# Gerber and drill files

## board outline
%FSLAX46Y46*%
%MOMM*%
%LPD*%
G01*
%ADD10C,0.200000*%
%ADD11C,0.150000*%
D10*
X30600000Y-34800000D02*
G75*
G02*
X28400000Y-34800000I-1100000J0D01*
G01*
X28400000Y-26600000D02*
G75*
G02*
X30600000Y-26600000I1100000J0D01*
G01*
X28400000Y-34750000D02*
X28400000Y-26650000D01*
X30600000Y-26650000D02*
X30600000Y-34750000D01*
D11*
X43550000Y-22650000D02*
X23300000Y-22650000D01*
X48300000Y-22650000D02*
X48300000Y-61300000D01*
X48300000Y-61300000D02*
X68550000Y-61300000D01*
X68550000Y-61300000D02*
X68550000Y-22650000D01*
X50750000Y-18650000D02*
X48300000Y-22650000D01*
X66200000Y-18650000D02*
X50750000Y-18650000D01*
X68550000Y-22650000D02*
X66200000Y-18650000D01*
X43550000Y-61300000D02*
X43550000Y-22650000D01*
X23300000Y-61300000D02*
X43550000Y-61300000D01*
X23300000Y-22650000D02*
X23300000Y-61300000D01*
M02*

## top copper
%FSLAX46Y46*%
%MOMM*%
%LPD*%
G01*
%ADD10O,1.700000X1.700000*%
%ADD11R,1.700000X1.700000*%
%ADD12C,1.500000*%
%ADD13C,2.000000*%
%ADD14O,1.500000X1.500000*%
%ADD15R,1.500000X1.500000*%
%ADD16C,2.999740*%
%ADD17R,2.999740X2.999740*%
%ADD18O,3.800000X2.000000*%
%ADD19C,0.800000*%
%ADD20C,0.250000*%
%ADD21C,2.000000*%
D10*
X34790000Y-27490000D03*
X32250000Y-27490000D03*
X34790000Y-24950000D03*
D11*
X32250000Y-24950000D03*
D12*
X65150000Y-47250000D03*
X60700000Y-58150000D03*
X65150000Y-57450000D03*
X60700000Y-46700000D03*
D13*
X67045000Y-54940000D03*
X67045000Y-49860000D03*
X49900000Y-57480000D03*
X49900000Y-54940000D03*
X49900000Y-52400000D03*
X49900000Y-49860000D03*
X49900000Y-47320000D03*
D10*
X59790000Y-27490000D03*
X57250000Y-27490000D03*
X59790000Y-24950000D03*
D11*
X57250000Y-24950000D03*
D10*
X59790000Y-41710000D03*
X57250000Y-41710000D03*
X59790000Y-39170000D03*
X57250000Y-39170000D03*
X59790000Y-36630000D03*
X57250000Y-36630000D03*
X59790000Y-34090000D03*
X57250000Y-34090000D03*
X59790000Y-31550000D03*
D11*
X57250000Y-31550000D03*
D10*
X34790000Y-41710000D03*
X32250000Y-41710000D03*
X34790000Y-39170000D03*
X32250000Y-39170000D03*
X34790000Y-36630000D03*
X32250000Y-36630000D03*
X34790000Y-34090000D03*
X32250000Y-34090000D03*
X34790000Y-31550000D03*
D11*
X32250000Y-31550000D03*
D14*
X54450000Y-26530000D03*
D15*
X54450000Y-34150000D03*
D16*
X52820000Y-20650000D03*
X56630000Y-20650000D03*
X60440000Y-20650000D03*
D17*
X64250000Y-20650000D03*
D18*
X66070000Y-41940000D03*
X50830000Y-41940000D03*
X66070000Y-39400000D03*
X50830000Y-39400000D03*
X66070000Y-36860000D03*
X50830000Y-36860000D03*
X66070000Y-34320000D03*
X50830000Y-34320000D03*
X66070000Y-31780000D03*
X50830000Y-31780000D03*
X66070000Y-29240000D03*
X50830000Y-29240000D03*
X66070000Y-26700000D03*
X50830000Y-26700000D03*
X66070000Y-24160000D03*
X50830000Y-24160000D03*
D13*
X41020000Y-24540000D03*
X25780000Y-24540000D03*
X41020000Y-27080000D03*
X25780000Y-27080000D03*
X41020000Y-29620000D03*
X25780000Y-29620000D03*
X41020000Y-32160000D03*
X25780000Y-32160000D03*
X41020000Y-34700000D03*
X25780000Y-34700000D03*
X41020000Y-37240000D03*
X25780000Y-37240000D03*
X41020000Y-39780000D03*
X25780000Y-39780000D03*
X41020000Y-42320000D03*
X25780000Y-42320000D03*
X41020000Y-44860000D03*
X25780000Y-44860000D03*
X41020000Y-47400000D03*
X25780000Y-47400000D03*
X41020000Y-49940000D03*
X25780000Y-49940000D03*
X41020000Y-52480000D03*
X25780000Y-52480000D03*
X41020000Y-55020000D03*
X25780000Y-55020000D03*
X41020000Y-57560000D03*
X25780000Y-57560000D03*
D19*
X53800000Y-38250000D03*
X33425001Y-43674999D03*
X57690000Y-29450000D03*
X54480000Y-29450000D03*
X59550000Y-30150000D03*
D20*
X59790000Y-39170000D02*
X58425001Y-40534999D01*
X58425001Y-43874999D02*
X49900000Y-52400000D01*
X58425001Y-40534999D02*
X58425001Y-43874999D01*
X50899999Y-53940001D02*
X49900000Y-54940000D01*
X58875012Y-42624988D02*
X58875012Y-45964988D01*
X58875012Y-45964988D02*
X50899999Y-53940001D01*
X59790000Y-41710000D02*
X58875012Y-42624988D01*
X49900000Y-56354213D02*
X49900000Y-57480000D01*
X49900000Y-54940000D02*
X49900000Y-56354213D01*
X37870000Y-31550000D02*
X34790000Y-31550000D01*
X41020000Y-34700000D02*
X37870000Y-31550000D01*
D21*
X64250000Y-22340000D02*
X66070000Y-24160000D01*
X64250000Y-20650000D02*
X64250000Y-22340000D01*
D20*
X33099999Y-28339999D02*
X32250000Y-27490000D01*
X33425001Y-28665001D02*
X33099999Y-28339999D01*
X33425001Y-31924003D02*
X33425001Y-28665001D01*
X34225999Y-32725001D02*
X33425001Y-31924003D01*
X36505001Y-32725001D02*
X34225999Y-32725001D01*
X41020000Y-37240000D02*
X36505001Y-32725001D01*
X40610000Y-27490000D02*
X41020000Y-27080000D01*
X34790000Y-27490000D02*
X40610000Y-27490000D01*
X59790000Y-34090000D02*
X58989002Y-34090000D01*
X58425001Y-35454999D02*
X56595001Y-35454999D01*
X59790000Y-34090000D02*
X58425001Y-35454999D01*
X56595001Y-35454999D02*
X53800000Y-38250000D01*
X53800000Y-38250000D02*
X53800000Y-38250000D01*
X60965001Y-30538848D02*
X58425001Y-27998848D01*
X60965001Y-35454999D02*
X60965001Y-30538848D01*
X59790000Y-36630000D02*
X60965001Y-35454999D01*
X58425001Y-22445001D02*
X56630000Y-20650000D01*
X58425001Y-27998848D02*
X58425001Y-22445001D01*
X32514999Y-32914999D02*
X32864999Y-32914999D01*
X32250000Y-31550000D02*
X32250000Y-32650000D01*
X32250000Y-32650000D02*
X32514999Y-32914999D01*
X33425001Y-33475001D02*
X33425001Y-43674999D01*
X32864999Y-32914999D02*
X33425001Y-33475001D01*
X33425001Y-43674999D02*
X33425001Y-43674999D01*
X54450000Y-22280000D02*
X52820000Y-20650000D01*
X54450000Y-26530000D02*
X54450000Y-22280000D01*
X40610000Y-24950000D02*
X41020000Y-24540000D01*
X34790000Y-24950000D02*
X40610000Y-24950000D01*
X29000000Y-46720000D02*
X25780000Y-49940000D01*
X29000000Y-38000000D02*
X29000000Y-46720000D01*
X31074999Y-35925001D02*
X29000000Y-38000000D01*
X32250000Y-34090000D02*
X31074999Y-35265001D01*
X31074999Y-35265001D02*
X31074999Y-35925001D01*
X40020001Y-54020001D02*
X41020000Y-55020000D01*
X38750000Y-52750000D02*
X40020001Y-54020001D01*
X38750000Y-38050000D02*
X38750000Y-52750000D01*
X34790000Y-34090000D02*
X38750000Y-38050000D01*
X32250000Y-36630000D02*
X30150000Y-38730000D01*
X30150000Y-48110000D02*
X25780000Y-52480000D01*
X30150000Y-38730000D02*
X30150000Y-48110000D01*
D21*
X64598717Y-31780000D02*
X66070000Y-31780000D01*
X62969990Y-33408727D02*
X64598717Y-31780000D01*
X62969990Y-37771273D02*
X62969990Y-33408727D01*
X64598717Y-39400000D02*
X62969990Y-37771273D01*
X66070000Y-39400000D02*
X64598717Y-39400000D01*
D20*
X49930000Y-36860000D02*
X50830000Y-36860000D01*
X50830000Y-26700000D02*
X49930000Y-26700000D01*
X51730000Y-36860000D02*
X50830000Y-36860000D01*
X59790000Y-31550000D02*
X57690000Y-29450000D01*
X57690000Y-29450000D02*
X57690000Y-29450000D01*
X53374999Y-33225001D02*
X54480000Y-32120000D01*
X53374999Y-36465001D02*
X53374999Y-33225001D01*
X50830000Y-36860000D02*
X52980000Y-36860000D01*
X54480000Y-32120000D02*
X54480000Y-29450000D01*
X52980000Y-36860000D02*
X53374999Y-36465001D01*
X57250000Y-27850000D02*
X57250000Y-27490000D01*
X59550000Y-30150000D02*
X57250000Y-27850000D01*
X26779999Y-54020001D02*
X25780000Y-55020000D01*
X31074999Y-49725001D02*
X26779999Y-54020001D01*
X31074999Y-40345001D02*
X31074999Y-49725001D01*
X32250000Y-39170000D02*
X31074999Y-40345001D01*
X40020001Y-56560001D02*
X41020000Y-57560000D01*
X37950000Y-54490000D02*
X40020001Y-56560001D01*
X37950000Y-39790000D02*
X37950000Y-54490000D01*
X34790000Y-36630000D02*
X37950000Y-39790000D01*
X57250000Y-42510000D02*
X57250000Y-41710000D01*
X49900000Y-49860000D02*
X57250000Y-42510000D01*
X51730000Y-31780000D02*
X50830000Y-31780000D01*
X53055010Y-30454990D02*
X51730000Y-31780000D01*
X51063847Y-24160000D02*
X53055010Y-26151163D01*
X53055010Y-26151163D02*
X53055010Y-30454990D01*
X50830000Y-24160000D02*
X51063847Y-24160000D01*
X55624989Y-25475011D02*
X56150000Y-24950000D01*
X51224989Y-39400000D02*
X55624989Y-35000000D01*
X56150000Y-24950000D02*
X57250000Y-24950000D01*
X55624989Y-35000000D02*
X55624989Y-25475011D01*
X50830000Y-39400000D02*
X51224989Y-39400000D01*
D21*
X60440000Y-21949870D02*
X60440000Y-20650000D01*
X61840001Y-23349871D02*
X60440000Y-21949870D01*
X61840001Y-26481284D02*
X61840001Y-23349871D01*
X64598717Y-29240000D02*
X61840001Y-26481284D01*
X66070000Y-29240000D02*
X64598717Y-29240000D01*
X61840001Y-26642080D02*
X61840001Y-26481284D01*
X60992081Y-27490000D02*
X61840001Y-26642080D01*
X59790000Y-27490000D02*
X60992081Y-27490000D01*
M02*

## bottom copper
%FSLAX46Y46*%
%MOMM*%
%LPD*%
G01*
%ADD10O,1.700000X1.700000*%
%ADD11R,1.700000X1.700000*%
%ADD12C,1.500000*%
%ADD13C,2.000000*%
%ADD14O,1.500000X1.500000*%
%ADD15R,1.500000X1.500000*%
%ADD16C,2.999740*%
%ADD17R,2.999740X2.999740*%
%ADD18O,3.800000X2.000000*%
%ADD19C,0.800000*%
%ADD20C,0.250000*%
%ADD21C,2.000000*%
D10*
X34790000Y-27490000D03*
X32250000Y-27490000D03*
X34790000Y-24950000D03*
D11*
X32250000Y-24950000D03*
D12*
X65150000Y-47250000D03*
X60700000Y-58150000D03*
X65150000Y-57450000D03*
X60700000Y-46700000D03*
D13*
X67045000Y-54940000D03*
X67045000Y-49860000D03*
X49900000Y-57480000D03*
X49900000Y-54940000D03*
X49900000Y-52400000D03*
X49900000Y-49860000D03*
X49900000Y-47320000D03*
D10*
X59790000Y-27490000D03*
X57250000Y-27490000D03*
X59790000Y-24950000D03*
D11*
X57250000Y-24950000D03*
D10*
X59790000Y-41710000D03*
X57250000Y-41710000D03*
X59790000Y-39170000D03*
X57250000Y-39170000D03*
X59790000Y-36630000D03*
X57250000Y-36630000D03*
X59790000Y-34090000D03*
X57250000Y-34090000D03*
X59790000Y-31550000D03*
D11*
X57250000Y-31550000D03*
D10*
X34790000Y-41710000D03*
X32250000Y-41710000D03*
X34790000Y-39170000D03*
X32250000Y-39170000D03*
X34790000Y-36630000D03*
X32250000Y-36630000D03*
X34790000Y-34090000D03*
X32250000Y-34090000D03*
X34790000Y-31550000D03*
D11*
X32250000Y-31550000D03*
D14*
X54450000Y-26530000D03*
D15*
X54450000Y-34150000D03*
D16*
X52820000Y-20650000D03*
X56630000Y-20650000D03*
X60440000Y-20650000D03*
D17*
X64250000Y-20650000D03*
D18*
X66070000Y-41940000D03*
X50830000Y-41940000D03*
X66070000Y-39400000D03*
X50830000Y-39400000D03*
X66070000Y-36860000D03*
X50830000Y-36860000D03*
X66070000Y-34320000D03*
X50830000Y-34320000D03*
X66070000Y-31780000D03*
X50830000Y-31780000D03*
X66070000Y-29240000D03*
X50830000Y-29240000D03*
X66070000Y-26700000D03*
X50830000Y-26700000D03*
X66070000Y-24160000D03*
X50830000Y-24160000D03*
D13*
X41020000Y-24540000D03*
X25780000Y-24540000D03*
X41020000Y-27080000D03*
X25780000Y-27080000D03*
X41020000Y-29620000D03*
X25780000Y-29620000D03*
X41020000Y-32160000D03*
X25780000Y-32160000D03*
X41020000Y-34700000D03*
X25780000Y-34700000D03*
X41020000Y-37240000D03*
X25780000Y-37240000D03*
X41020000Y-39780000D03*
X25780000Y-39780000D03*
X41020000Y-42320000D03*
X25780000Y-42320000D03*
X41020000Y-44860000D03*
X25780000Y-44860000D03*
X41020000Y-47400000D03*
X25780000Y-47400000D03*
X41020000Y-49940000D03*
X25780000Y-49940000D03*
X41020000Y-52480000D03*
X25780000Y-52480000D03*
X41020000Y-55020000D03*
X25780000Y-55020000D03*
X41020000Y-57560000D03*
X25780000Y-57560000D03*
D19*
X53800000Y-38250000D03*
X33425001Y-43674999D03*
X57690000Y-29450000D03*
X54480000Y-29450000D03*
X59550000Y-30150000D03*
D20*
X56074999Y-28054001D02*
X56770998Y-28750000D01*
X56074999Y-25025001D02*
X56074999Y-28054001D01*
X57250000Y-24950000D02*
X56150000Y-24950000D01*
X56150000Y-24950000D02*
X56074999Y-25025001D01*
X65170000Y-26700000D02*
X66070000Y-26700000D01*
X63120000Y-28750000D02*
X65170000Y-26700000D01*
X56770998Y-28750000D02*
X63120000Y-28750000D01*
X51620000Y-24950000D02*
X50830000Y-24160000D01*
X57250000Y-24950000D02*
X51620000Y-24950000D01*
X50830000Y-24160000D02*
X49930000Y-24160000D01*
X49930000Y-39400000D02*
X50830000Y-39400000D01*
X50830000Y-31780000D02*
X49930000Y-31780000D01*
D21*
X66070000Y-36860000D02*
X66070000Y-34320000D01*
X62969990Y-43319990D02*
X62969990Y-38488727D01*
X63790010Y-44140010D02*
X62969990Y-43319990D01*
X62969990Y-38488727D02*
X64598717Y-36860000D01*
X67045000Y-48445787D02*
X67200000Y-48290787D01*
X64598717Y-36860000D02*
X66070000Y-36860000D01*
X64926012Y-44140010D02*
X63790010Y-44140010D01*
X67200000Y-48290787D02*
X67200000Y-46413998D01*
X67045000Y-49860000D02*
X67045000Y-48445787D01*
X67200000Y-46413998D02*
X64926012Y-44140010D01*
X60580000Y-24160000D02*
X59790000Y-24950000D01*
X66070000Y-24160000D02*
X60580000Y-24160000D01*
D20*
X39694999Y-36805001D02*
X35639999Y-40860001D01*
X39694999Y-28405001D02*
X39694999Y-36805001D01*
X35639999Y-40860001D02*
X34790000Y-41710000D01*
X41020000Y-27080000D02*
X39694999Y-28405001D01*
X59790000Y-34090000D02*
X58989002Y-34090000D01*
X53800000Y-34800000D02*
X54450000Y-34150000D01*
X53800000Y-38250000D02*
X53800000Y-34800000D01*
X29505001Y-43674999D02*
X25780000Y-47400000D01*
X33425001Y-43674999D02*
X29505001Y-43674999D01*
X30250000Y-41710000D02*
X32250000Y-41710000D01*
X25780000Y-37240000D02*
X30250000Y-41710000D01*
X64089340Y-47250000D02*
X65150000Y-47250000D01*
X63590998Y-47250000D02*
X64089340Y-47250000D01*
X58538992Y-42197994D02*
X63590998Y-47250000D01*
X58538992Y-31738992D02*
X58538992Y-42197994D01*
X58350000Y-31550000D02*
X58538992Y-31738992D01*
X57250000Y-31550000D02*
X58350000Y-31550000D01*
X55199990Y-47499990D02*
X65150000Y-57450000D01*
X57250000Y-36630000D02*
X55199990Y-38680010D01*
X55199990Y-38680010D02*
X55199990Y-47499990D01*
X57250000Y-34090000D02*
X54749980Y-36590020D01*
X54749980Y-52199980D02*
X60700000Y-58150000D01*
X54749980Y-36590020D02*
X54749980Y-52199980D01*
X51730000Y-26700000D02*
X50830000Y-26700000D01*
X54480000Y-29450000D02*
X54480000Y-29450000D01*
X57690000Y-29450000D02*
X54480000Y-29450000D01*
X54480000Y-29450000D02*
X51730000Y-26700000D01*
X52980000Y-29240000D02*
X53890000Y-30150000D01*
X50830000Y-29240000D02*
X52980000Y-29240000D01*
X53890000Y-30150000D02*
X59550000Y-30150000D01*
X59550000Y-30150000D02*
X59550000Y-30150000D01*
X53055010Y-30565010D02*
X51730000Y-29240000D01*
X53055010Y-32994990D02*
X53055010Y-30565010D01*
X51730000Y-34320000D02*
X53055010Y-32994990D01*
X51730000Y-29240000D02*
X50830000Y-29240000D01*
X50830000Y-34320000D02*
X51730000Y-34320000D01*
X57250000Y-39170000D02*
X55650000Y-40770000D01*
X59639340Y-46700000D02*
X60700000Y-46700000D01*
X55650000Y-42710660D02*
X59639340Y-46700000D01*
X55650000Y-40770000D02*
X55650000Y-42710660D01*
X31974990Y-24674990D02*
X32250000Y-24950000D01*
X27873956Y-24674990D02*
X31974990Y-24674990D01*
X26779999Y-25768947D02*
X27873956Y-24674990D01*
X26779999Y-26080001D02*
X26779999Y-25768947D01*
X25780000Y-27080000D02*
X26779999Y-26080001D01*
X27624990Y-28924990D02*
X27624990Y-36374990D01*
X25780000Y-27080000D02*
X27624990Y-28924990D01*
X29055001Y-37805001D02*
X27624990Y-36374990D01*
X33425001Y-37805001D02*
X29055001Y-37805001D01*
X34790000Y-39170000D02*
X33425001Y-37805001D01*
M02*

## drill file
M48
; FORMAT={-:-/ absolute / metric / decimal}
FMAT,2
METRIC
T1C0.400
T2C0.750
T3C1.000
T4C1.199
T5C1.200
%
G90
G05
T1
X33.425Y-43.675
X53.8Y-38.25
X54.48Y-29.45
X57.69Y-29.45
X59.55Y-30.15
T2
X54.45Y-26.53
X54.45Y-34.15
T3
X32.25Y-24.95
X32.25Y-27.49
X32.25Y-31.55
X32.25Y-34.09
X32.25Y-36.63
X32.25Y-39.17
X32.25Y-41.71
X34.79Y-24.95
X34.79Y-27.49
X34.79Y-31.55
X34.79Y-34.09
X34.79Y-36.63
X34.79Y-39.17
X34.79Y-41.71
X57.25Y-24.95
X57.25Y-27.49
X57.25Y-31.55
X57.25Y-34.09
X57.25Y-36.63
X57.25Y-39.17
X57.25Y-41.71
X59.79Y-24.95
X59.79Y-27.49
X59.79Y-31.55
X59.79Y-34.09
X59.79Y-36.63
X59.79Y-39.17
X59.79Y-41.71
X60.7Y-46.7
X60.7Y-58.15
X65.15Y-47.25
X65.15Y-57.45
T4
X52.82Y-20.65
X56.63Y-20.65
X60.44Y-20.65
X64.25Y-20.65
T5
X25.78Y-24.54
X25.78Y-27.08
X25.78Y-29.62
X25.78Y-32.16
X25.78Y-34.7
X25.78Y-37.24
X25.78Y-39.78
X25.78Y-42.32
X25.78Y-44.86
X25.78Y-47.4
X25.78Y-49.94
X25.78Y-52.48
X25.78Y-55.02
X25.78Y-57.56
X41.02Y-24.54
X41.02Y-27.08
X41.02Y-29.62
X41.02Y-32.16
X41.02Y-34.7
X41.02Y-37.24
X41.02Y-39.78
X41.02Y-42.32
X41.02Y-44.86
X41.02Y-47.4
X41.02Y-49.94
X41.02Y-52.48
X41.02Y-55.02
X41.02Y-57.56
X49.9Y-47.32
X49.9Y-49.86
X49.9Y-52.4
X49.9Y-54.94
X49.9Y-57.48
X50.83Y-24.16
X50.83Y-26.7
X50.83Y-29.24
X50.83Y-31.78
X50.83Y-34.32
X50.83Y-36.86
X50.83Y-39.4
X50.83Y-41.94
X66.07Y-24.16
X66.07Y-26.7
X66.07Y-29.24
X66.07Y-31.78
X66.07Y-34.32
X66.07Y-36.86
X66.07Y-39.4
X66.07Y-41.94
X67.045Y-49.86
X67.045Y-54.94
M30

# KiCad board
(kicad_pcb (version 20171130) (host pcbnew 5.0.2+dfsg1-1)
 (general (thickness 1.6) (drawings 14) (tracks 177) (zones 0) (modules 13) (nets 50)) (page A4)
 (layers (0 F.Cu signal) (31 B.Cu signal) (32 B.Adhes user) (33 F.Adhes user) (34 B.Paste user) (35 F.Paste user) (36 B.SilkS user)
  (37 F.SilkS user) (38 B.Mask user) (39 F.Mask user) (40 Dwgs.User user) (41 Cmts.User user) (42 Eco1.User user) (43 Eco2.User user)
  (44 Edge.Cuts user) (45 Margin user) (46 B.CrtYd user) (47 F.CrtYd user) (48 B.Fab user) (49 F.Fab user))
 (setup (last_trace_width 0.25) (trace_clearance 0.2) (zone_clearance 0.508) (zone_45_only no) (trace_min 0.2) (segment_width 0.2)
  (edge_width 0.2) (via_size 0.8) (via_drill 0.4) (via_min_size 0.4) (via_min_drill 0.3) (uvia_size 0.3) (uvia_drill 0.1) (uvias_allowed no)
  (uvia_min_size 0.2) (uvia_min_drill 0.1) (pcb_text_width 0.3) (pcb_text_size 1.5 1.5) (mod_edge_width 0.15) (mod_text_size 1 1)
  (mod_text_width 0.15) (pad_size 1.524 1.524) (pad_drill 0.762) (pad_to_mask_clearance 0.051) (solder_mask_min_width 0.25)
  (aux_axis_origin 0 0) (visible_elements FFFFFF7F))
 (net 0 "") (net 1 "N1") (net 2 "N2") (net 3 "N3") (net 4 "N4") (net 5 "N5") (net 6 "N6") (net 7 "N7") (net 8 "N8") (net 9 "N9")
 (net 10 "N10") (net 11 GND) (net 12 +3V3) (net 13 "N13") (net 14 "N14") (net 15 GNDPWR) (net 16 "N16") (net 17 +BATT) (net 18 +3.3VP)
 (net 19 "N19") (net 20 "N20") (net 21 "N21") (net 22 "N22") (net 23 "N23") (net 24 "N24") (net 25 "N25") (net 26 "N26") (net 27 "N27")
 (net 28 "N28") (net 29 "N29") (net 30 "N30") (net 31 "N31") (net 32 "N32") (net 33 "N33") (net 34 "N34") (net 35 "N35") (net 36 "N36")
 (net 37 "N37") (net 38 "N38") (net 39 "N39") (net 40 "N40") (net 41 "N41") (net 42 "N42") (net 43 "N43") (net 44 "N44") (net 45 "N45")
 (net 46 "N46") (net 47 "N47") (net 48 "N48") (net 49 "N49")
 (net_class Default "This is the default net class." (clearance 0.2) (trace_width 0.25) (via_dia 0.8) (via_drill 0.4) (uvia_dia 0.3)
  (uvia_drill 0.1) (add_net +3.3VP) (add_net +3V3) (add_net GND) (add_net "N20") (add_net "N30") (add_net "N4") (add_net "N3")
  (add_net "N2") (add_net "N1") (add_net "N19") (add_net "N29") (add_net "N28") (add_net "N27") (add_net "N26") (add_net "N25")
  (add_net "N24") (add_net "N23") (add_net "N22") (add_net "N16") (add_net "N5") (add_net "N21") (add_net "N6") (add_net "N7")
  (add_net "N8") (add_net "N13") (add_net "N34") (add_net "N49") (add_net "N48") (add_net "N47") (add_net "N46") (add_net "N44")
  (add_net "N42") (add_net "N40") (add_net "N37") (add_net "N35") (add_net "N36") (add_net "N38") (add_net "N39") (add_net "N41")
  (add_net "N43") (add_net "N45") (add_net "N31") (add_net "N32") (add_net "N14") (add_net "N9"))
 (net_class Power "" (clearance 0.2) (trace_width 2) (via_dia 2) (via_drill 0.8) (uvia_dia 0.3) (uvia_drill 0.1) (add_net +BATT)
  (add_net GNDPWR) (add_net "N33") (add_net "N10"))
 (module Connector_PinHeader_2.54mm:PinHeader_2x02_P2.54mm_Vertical (layer F.Cu) (at 32.25 24.95)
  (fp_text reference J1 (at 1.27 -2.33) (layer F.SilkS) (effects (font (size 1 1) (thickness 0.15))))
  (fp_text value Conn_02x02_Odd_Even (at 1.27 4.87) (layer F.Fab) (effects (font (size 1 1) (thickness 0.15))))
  (pad 4 thru_hole oval (at 2.54 2.54) (size 1.7 1.7) (drill 1) (layers *.Cu *.Mask) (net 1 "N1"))
  (pad 3 thru_hole oval (at 0 2.54) (size 1.7 1.7) (drill 1) (layers *.Cu *.Mask) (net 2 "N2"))
  (pad 2 thru_hole oval (at 2.54 0) (size 1.7 1.7) (drill 1) (layers *.Cu *.Mask) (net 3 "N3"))
  (pad 1 thru_hole rect (at 0 0) (size 1.7 1.7) (drill 1) (layers *.Cu *.Mask) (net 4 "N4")))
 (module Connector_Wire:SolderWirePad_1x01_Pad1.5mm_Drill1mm (layer B.Cu) (at 65.15 47.25)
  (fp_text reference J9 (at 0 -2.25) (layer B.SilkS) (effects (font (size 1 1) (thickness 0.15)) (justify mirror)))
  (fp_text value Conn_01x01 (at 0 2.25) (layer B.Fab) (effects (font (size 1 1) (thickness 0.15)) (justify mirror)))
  (pad 1 thru_hole circle (at 0 0) (size 1.5 1.5) (drill 1) (layers *.Cu *.Mask) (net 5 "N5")))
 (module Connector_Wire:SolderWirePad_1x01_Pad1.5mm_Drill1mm (layer B.Cu) (at 60.7 58.15)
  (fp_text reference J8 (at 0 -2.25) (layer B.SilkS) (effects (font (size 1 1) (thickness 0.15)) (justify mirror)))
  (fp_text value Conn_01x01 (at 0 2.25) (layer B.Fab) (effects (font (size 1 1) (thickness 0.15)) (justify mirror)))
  (pad 1 thru_hole circle (at 0 0) (size 1.5 1.5) (drill 1) (layers *.Cu *.Mask) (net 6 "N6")))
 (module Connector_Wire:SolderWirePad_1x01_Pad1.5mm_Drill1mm (layer B.Cu) (at 65.15 57.45)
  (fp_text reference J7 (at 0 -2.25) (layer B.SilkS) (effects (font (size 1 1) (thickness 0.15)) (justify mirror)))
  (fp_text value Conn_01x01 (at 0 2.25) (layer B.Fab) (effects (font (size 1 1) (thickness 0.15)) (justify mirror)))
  (pad 1 thru_hole circle (at 0 0) (size 1.5 1.5) (drill 1) (layers *.Cu *.Mask) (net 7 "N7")))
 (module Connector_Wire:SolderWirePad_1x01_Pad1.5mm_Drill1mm (layer B.Cu) (at 60.7 46.7)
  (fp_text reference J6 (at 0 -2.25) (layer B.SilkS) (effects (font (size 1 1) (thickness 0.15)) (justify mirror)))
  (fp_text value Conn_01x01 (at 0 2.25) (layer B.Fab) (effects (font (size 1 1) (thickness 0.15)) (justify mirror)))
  (pad 1 thru_hole circle (at 0 0) (size 1.5 1.5) (drill 1) (layers *.Cu *.Mask) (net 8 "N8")))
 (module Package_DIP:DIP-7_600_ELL (layer B.Cu) (at 49.9 52.4 270)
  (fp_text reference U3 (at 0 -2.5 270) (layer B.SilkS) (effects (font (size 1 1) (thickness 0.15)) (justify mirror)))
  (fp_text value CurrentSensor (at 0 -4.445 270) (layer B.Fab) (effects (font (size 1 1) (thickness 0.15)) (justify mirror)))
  (pad 7 thru_hole circle (at 2.54 -17.145 270) (size 2 2) (drill 1.2) (layers *.Cu *.Mask) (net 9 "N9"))
  (pad 6 thru_hole circle (at -2.54 -17.145 270) (size 2 2) (drill 1.2) (layers *.Cu *.Mask) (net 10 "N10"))
  (pad 5 thru_hole circle (at 5.08 0 270) (size 2 2) (drill 1.2) (layers *.Cu *.Mask) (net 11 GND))
  (pad 4 thru_hole circle (at 2.54 0 270) (size 2 2) (drill 1.2) (layers *.Cu *.Mask) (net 11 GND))
  (pad 3 thru_hole circle (at 0 0 270) (size 2 2) (drill 1.2) (layers *.Cu *.Mask) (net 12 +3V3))
  (pad 2 thru_hole circle (at -2.54 0 270) (size 2 2) (drill 1.2) (layers *.Cu *.Mask) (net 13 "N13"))
  (pad 1 thru_hole circle (at -5.08 0 270) (size 2 2) (drill 1.2) (layers *.Cu *.Mask) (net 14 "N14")))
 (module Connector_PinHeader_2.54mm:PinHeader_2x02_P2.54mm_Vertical (layer F.Cu) (at 57.25 24.95)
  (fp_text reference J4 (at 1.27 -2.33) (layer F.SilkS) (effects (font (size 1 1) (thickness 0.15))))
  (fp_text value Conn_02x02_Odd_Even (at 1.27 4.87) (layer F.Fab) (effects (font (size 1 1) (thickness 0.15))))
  (pad 4 thru_hole oval (at 2.54 2.54) (size 1.7 1.7) (drill 1) (layers *.Cu *.Mask) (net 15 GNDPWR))
  (pad 3 thru_hole oval (at 0 2.54) (size 1.7 1.7) (drill 1) (layers *.Cu *.Mask) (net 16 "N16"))
  (pad 2 thru_hole oval (at 2.54 0) (size 1.7 1.7) (drill 1) (layers *.Cu *.Mask) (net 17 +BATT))
  (pad 1 thru_hole rect (at 0 0) (size 1.7 1.7) (drill 1) (layers *.Cu *.Mask) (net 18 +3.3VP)))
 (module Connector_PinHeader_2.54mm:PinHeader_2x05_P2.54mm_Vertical (layer F.Cu) (at 57.25 31.55)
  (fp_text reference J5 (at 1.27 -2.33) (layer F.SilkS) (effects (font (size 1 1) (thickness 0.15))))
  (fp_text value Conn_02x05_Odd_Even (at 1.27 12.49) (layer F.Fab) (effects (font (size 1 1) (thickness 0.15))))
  (pad 10 thru_hole oval (at 2.54 10.16) (size 1.7 1.7) (drill 1) (layers *.Cu *.Mask) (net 11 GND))
  (pad 9 thru_hole oval (at 0 10.16) (size 1.7 1.7) (drill 1) (layers *.Cu *.Mask) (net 13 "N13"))
  (pad 8 thru_hole oval (at 2.54 7.62) (size 1.7 1.7) (drill 1) (layers *.Cu *.Mask) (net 12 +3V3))
  (pad 7 thru_hole oval (at 0 7.62) (size 1.7 1.7) (drill 1) (layers *.Cu *.Mask) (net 8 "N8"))
  (pad 6 thru_hole oval (at 2.54 5.08) (size 1.7 1.7) (drill 1) (layers *.Cu *.Mask) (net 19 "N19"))
  (pad 5 thru_hole oval (at 0 5.08) (size 1.7 1.7) (drill 1) (layers *.Cu *.Mask) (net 7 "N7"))
  (pad 4 thru_hole oval (at 2.54 2.54) (size 1.7 1.7) (drill 1) (layers *.Cu *.Mask) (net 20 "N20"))
  (pad 3 thru_hole oval (at 0 2.54) (size 1.7 1.7) (drill 1) (layers *.Cu *.Mask) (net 6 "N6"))
  (pad 2 thru_hole oval (at 2.54 0) (size 1.7 1.7) (drill 1) (layers *.Cu *.Mask) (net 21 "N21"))
  (pad 1 thru_hole rect (at 0 0) (size 1.7 1.7) (drill 1) (layers *.Cu *.Mask) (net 5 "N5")))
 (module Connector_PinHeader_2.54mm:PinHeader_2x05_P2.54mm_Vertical (layer F.Cu) (at 32.25 31.55)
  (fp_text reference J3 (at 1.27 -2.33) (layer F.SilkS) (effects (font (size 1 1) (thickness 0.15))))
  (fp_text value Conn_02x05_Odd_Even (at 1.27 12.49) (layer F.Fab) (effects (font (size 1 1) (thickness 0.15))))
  (pad 10 thru_hole oval (at 2.54 10.16) (size 1.7 1.7) (drill 1) (layers *.Cu *.Mask) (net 1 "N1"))
  (pad 9 thru_hole oval (at 0 10.16) (size 1.7 1.7) (drill 1) (layers *.Cu *.Mask) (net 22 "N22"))
  (pad 8 thru_hole oval (at 2.54 7.62) (size 1.7 1.7) (drill 1) (layers *.Cu *.Mask) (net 4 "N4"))
  (pad 7 thru_hole oval (at 0 7.62) (size 1.7 1.7) (drill 1) (layers *.Cu *.Mask) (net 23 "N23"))
  (pad 6 thru_hole oval (at 2.54 5.08) (size 1.7 1.7) (drill 1) (layers *.Cu *.Mask) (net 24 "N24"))
  (pad 5 thru_hole oval (at 0 5.08) (size 1.7 1.7) (drill 1) (layers *.Cu *.Mask) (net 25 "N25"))
  (pad 4 thru_hole oval (at 2.54 2.54) (size 1.7 1.7) (drill 1) (layers *.Cu *.Mask) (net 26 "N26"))
  (pad 3 thru_hole oval (at 0 2.54) (size 1.7 1.7) (drill 1) (layers *.Cu *.Mask) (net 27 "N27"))
  (pad 2 thru_hole oval (at 2.54 0) (size 1.7 1.7) (drill 1) (layers *.Cu *.Mask) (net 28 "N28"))
  (pad 1 thru_hole rect (at 0 0) (size 1.7 1.7) (drill 1) (layers *.Cu *.Mask) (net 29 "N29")))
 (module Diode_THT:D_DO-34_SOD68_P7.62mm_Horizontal (layer F.Cu) (at 54.45 34.15 90)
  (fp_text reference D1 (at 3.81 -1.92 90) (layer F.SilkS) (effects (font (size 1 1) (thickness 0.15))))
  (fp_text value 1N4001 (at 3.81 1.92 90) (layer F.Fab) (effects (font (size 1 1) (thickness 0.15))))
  (pad 2 thru_hole oval (at 7.62 0 90) (size 1.5 1.5) (drill 0.75) (layers *.Cu *.Mask) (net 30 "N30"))
  (pad 1 thru_hole rect (at 0 0 90) (size 1.5 1.5) (drill 0.75) (layers *.Cu *.Mask) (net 20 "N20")))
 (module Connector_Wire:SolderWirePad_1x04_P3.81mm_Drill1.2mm (layer F.Cu) (at 64.25 20.65 180)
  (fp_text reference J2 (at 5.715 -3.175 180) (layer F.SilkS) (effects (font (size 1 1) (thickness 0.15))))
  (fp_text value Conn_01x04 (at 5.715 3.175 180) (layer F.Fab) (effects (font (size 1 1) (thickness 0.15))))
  (pad 4 thru_hole circle (at 11.43 0 180) (size 2.99974 2.99974) (drill 1.19888) (layers *.Cu *.Mask) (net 30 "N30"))
  (pad 3 thru_hole circle (at 7.62 0 180) (size 2.99974 2.99974) (drill 1.19888) (layers *.Cu *.Mask) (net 19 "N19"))
  (pad 2 thru_hole circle (at 3.81 0 180) (size 2.99974 2.99974) (drill 1.19888) (layers *.Cu *.Mask) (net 15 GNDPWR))
  (pad 1 thru_hole rect (at 0 0 180) (size 2.99974 2.99974) (drill 1.19888) (layers *.Cu *.Mask) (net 17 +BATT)))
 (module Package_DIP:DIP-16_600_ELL (layer B.Cu) (at 58.45 33.05 270)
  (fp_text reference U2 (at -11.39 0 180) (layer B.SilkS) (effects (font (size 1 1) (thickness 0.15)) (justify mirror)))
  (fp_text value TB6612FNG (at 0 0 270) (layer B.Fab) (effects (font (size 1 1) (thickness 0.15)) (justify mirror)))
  (pad 8 thru_hole oval (at 8.89 -7.62 270) (size 2 3.8) (drill 1.2) (layers *.Cu *.Mask) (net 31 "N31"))
  (pad 9 thru_hole oval (at 8.89 7.62 270) (size 2 3.8) (drill 1.2) (layers *.Cu *.Mask) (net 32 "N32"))
  (pad 7 thru_hole oval (at 6.35 -7.62 270) (size 2 3.8) (drill 1.2) (layers *.Cu *.Mask) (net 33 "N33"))
  (pad 10 thru_hole oval (at 6.35 7.62 270) (size 2 3.8) (drill 1.2) (layers *.Cu *.Mask) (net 18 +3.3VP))
  (pad 6 thru_hole oval (at 3.81 -7.62 270) (size 2 3.8) (drill 1.2) (layers *.Cu *.Mask) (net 10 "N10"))
  (pad 11 thru_hole oval (at 3.81 7.62 270) (size 2 3.8) (drill 1.2) (layers *.Cu *.Mask) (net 21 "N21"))
  (pad 5 thru_hole oval (at 1.27 -7.62 270) (size 2 3.8) (drill 1.2) (layers *.Cu *.Mask) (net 10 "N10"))
  (pad 12 thru_hole oval (at 1.27 7.62 270) (size 2 3.8) (drill 1.2) (layers *.Cu *.Mask) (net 16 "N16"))
  (pad 4 thru_hole oval (at -1.27 -7.62 270) (size 2 3.8) (drill 1.2) (layers *.Cu *.Mask) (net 33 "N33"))
  (pad 13 thru_hole oval (at -1.27 7.62 270) (size 2 3.8) (drill 1.2) (layers *.Cu *.Mask) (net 18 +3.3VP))
  (pad 3 thru_hole oval (at -3.81 -7.62 270) (size 2 3.8) (drill 1.2) (layers *.Cu *.Mask) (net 15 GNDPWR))
  (pad 14 thru_hole oval (at -3.81 7.62 270) (size 2 3.8) (drill 1.2) (layers *.Cu *.Mask) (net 16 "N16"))
  (pad 2 thru_hole oval (at -6.35 -7.62 270) (size 2 3.8) (drill 1.2) (layers *.Cu *.Mask) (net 18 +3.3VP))
  (pad 15 thru_hole oval (at -6.35 7.62 270) (size 2 3.8) (drill 1.2) (layers *.Cu *.Mask) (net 21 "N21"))
  (pad 1 thru_hole oval (at -8.89 -7.62 270) (size 2 3.8) (drill 1.2) (layers *.Cu *.Mask) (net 17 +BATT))
  (pad 16 thru_hole oval (at -8.89 7.62 270) (size 2 3.8) (drill 1.2) (layers *.Cu *.Mask) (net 18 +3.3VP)))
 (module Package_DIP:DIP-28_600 (layer F.Cu) (at 33.4 41.05 270)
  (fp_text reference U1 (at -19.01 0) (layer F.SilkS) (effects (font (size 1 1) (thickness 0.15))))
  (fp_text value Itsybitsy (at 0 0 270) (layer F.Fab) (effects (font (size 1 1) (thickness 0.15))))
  (pad 28 thru_hole circle (at -16.51 -7.62 270) (size 2 2) (drill 1.2) (layers *.Cu *.Mask) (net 3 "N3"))
  (pad 1 thru_hole circle (at -16.51 7.62 270) (size 2 2) (drill 1.2) (layers *.Cu *.Mask) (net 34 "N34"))
  (pad 27 thru_hole circle (at -13.97 -7.62 270) (size 2 2) (drill 1.2) (layers *.Cu *.Mask) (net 1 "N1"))
  (pad 2 thru_hole circle (at -13.97 7.62 270) (size 2 2) (drill 1.2) (layers *.Cu *.Mask) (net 4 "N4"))
  (pad 26 thru_hole circle (at -11.43 -7.62 270) (size 2 2) (drill 1.2) (layers *.Cu *.Mask) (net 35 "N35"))
  (pad 3 thru_hole circle (at -11.43 7.62 270) (size 2 2) (drill 1.2) (layers *.Cu *.Mask) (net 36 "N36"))
  (pad 25 thru_hole circle (at -8.89 -7.62 270) (size 2 2) (drill 1.2) (layers *.Cu *.Mask) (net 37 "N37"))
  (pad 4 thru_hole circle (at -8.89 7.62 270) (size 2 2) (drill 1.2) (layers *.Cu *.Mask) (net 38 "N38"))
  (pad 24 thru_hole circle (at -6.35 -7.62 270) (size 2 2) (drill 1.2) (layers *.Cu *.Mask) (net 28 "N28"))
  (pad 5 thru_hole circle (at -6.35 7.62 270) (size 2 2) (drill 1.2) (layers *.Cu *.Mask) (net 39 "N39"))
  (pad 23 thru_hole circle (at -3.81 -7.62 270) (size 2 2) (drill 1.2) (layers *.Cu *.Mask) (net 2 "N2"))
  (pad 6 thru_hole circle (at -3.81 7.62 270) (size 2 2) (drill 1.2) (layers *.Cu *.Mask) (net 22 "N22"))
  (pad 22 thru_hole circle (at -1.27 -7.62 270) (size 2 2) (drill 1.2) (layers *.Cu *.Mask) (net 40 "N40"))
  (pad 7 thru_hole circle (at -1.27 7.62 270) (size 2 2) (drill 1.2) (layers *.Cu *.Mask) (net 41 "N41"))
  (pad 21 thru_hole circle (at 1.27 -7.62 270) (size 2 2) (drill 1.2) (layers *.Cu *.Mask) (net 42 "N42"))
  (pad 8 thru_hole circle (at 1.27 7.62 270) (size 2 2) (drill 1.2) (layers *.Cu *.Mask) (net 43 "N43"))
  (pad 20 thru_hole circle (at 3.81 -7.62 270) (size 2 2) (drill 1.2) (layers *.Cu *.Mask) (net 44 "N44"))
  (pad 9 thru_hole circle (at 3.81 7.62 270) (size 2 2) (drill 1.2) (layers *.Cu *.Mask) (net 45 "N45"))
  (pad 19 thru_hole circle (at 6.35 -7.62 270) (size 2 2) (drill 1.2) (layers *.Cu *.Mask) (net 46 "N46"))
  (pad 10 thru_hole circle (at 6.35 7.62 270) (size 2 2) (drill 1.2) (layers *.Cu *.Mask) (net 29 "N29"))
  (pad 18 thru_hole circle (at 8.89 -7.62 270) (size 2 2) (drill 1.2) (layers *.Cu *.Mask) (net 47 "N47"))
  (pad 11 thru_hole circle (at 8.89 7.62 270) (size 2 2) (drill 1.2) (layers *.Cu *.Mask) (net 27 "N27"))
  (pad 17 thru_hole circle (at 11.43 -7.62 270) (size 2 2) (drill 1.2) (layers *.Cu *.Mask) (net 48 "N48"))
  (pad 12 thru_hole circle (at 11.43 7.62 270) (size 2 2) (drill 1.2) (layers *.Cu *.Mask) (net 25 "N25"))
  (pad 16 thru_hole circle (at 13.97 -7.62 270) (size 2 2) (drill 1.2) (layers *.Cu *.Mask) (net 26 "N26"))
  (pad 13 thru_hole circle (at 13.97 7.62 270) (size 2 2) (drill 1.2) (layers *.Cu *.Mask) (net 23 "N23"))
  (pad 15 thru_hole circle (at 16.51 -7.62 270) (size 2 2) (drill 1.2) (layers *.Cu *.Mask) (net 24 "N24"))
  (pad 14 thru_hole circle (at 16.51 7.62 270) (size 2 2) (drill 1.2) (layers *.Cu *.Mask) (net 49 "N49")))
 (gr_arc (start 29.5 34.8) (end 28.4 34.8) (angle -180) (layer Edge.Cuts) (width 0.2))
 (gr_arc (start 29.5 26.6) (end 30.6 26.6) (angle -180) (layer Edge.Cuts) (width 0.2))
 (gr_line (start 28.4 34.75) (end 28.4 26.65) (layer Edge.Cuts) (width 0.2))
 (gr_line (start 30.6 26.65) (end 30.6 34.75) (layer Edge.Cuts) (width 0.2))
 (gr_line (start 43.55 22.65) (end 23.3 22.65) (layer Edge.Cuts) (width 0.15))
 (gr_line (start 48.3 22.65) (end 48.3 61.3) (layer Edge.Cuts) (width 0.15))
 (gr_line (start 48.3 61.3) (end 68.55 61.3) (layer Edge.Cuts) (width 0.15))
 (gr_line (start 68.55 61.3) (end 68.55 22.65) (layer Edge.Cuts) (width 0.15))
 (gr_line (start 50.75 18.65) (end 48.3 22.65) (layer Edge.Cuts) (width 0.15))
 (gr_line (start 66.2 18.65) (end 50.75 18.65) (layer Edge.Cuts) (width 0.15))
 (gr_line (start 68.55 22.65) (end 66.2 18.65) (layer Edge.Cuts) (width 0.15))
 (gr_line (start 43.55 61.3) (end 43.55 22.65) (layer Edge.Cuts) (width 0.15))
 (gr_line (start 23.3 61.3) (end 43.55 61.3) (layer Edge.Cuts) (width 0.15))
 (gr_line (start 23.3 22.65) (end 23.3 61.3) (layer Edge.Cuts) (width 0.15))
 (segment (start 56.074999 28.054001) (end 56.770998 28.75) (width 0.25) (layer B.Cu) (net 18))
 (segment (start 56.074999 25.025001) (end 56.074999 28.054001) (width 0.25) (layer B.Cu) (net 18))
 (segment (start 57.25 24.95) (end 56.15 24.95) (width 0.25) (layer B.Cu) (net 18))
 (segment (start 56.15 24.95) (end 56.074999 25.025001) (width 0.25) (layer B.Cu) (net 18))
 (segment (start 65.17 26.7) (end 66.07 26.7) (width 0.25) (layer B.Cu) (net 18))
 (segment (start 63.12 28.75) (end 65.17 26.7) (width 0.25) (layer B.Cu) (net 18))
 (segment (start 56.770998 28.75) (end 63.12 28.75) (width 0.25) (layer B.Cu) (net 18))
 (segment (start 51.62 24.95) (end 50.83 24.16) (width 0.25) (layer B.Cu) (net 18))
 (segment (start 57.25 24.95) (end 51.62 24.95) (width 0.25) (layer B.Cu) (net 18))
 (segment (start 50.83 24.16) (end 49.93 24.16) (width 0.25) (layer B.Cu) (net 18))
 (segment (start 49.93 39.4) (end 50.83 39.4) (width 0.25) (layer B.Cu) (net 18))
 (segment (start 50.83 31.78) (end 49.93 31.78) (width 0.25) (layer B.Cu) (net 18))
 (segment (start 59.79 39.17) (end 58.425001 40.534999) (width 0.25) (layer F.Cu) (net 12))
 (segment (start 58.425001 43.874999) (end 49.9 52.4) (width 0.25) (layer F.Cu) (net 12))
 (segment (start 58.425001 40.534999) (end 58.425001 43.874999) (width 0.25) (layer F.Cu) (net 12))
 (segment (start 50.899999 53.940001) (end 49.9 54.94) (width 0.25) (layer F.Cu) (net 11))
 (segment (start 58.875012 42.624988) (end 58.875012 45.964988) (width 0.25) (layer F.Cu) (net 11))
 (segment (start 58.875012 45.964988) (end 50.899999 53.940001) (width 0.25) (layer F.Cu) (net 11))
 (segment (start 59.79 41.71) (end 58.875012 42.624988) (width 0.25) (layer F.Cu) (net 11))
 (segment (start 49.9 56.354213) (end 49.9 57.48) (width 0.25) (layer F.Cu) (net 11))
 (segment (start 49.9 54.94) (end 49.9 56.354213) (width 0.25) (layer F.Cu) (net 11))
 (segment (start 66.07 36.86) (end 66.07 34.32) (width 2) (layer B.Cu) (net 10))
 (segment (start 62.96999 43.31999) (end 62.96999 38.488727) (width 2) (layer B.Cu) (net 10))
 (segment (start 63.79001 44.14001) (end 62.96999 43.31999) (width 2) (layer B.Cu) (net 10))
 (segment (start 62.96999 38.488727) (end 64.598717 36.86) (width 2) (layer B.Cu) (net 10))
 (segment (start 67.045 48.445787) (end 67.2 48.290787) (width 2) (layer B.Cu) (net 10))
 (segment (start 64.598717 36.86) (end 66.07 36.86) (width 2) (layer B.Cu) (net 10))
 (segment (start 64.926012 44.14001) (end 63.79001 44.14001) (width 2) (layer B.Cu) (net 10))
 (segment (start 67.2 48.290787) (end 67.2 46.413998) (width 2) (layer B.Cu) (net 10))
 (segment (start 67.045 49.86) (end 67.045 48.445787) (width 2) (layer B.Cu) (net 10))
 (segment (start 67.2 46.413998) (end 64.926012 44.14001) (width 2) (layer B.Cu) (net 10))
 (segment (start 37.87 31.55) (end 34.79 31.55) (width 0.25) (layer F.Cu) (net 28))
 (segment (start 41.02 34.7) (end 37.87 31.55) (width 0.25) (layer F.Cu) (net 28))
 (segment (start 60.58 24.16) (end 59.79 24.95) (width 2) (layer B.Cu) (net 17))
 (segment (start 66.07 24.16) (end 60.58 24.16) (width 2) (layer B.Cu) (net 17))
 (segment (start 64.25 22.34) (end 66.07 24.16) (width 2) (layer F.Cu) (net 17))
 (segment (start 64.25 20.65) (end 64.25 22.34) (width 2) (layer F.Cu) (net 17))
 (segment (start 33.099999 28.339999) (end 32.25 27.49) (width 0.25) (layer F.Cu) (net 2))
 (segment (start 33.425001 28.665001) (end 33.099999 28.339999) (width 0.25) (layer F.Cu) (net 2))
 (segment (start 33.425001 31.924003) (end 33.425001 28.665001) (width 0.25) (layer F.Cu) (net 2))
 (segment (start 34.225999 32.725001) (end 33.425001 31.924003) (width 0.25) (layer F.Cu) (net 2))
 (segment (start 36.505001 32.725001) (end 34.225999 32.725001) (width 0.25) (layer F.Cu) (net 2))
 (segment (start 41.02 37.24) (end 36.505001 32.725001) (width 0.25) (layer F.Cu) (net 2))
 (segment (start 40.61 27.49) (end 41.02 27.08) (width 0.25) (layer F.Cu) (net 1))
 (segment (start 34.79 27.49) (end 40.61 27.49) (width 0.25) (layer F.Cu) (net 1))
 (segment (start 39.694999 36.805001) (end 35.639999 40.860001) (width 0.25) (layer B.Cu) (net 1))
 (segment (start 39.694999 28.405001) (end 39.694999 36.805001) (width 0.25) (layer B.Cu) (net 1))
 (segment (start 35.639999 40.860001) (end 34.79 41.71) (width 0.25) (layer B.Cu) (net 1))
 (segment (start 41.02 27.08) (end 39.694999 28.405001) (width 0.25) (layer B.Cu) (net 1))
 (segment (start 59.79 34.09) (end 58.989002 34.09) (width 0.25) (layer F.Cu) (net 20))
 (segment (start 59.79 34.09) (end 58.989002 34.09) (width 0.25) (layer B.Cu) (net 20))
 (segment (start 58.425001 35.454999) (end 56.595001 35.454999) (width 0.25) (layer F.Cu) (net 20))
 (segment (start 59.79 34.09) (end 58.425001 35.454999) (width 0.25) (layer F.Cu) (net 20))
 (segment (start 56.595001 35.454999) (end 53.8 38.25) (width 0.25) (layer F.Cu) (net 20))
 (segment (start 53.8 38.25) (end 53.8 38.25) (width 0.25) (layer F.Cu) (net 20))
 (via (at 53.8 38.25) (size 0.8) (drill 0.4) (layers F.Cu B.Cu) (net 20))
 (segment (start 53.8 34.8) (end 54.45 34.15) (width 0.25) (layer B.Cu) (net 20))
 (segment (start 53.8 38.25) (end 53.8 34.8) (width 0.25) (layer B.Cu) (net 20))
 (segment (start 60.965001 30.538848) (end 58.425001 27.998848) (width 0.25) (layer F.Cu) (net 19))
 (segment (start 60.965001 35.454999) (end 60.965001 30.538848) (width 0.25) (layer F.Cu) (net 19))
 (segment (start 59.79 36.63) (end 60.965001 35.454999) (width 0.25) (layer F.Cu) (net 19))
 (segment (start 58.425001 22.445001) (end 56.63 20.65) (width 0.25) (layer F.Cu) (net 19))
 (segment (start 58.425001 27.998848) (end 58.425001 22.445001) (width 0.25) (layer F.Cu) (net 19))
 (segment (start 32.514999 32.914999) (end 32.864999 32.914999) (width 0.25) (layer F.Cu) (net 29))
 (segment (start 32.25 31.55) (end 32.25 32.65) (width 0.25) (layer F.Cu) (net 29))
 (segment (start 32.25 32.65) (end 32.514999 32.914999) (width 0.25) (layer F.Cu) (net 29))
 (segment (start 33.425001 33.475001) (end 33.425001 43.674999) (width 0.25) (layer F.Cu) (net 29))
 (segment (start 32.864999 32.914999) (end 33.425001 33.475001) (width 0.25) (layer F.Cu) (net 29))
 (segment (start 33.425001 43.674999) (end 33.425001 43.674999) (width 0.25) (layer F.Cu) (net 29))
 (via (at 33.425001 43.674999) (size 0.8) (drill 0.4) (layers F.Cu B.Cu) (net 29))
 (segment (start 29.505001 43.674999) (end 25.78 47.4) (width 0.25) (layer B.Cu) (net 29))
 (segment (start 33.425001 43.674999) (end 29.505001 43.674999) (width 0.25) (layer B.Cu) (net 29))
 (segment (start 54.45 22.28) (end 52.82 20.65) (width 0.25) (layer F.Cu) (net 30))
 (segment (start 54.45 26.53) (end 54.45 22.28) (width 0.25) (layer F.Cu) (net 30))
 (segment (start 40.61 24.95) (end 41.02 24.54) (width 0.25) (layer F.Cu) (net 3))
 (segment (start 34.79 24.95) (end 40.61 24.95) (width 0.25) (layer F.Cu) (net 3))
 (segment (start 29 46.72) (end 25.78 49.94) (width 0.25) (layer F.Cu) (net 27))
 (segment (start 29 38) (end 29 46.72) (width 0.25) (layer F.Cu) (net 27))
 (segment (start 31.074999 35.925001) (end 29 38) (width 0.25) (layer F.Cu) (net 27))
 (segment (start 32.25 34.09) (end 31.074999 35.265001) (width 0.25) (layer F.Cu) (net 27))
 (segment (start 31.074999 35.265001) (end 31.074999 35.925001) (width 0.25) (layer F.Cu) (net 27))
 (segment (start 40.020001 54.020001) (end 41.02 55.02) (width 0.25) (layer F.Cu) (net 26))
 (segment (start 38.75 52.75) (end 40.020001 54.020001) (width 0.25) (layer F.Cu) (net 26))
 (segment (start 38.75 38.05) (end 38.75 52.75) (width 0.25) (layer F.Cu) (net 26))
 (segment (start 34.79 34.09) (end 38.75 38.05) (width 0.25) (layer F.Cu) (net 26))
 (segment (start 30.25 41.71) (end 32.25 41.71) (width 0.25) (layer B.Cu) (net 22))
 (segment (start 25.78 37.24) (end 30.25 41.71) (width 0.25) (layer B.Cu) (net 22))
 (segment (start 32.25 36.63) (end 30.15 38.73) (width 0.25) (layer F.Cu) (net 25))
 (segment (start 30.15 48.11) (end 25.78 52.48) (width 0.25) (layer F.Cu) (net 25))
 (segment (start 30.15 38.73) (end 30.15 48.11) (width 0.25) (layer F.Cu) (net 25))
 (segment (start 64.08934 47.25) (end 65.15 47.25) (width 0.25) (layer B.Cu) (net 5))
 (segment (start 63.590998 47.25) (end 64.08934 47.25) (width 0.25) (layer B.Cu) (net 5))
 (segment (start 58.538992 42.197994) (end 63.590998 47.25) (width 0.25) (layer B.Cu) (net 5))
 (segment (start 58.538992 31.738992) (end 58.538992 42.197994) (width 0.25) (layer B.Cu) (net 5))
 (segment (start 58.35 31.55) (end 58.538992 31.738992) (width 0.25) (layer B.Cu) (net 5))
 (segment (start 57.25 31.55) (end 58.35 31.55) (width 0.25) (layer B.Cu) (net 5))
 (segment (start 64.598717 31.78) (end 66.07 31.78) (width 2) (layer F.Cu) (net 33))
 (segment (start 62.96999 33.408727) (end 64.598717 31.78) (width 2) (layer F.Cu) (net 33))
 (segment (start 62.96999 37.771273) (end 62.96999 33.408727) (width 2) (layer F.Cu) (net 33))
 (segment (start 64.598717 39.4) (end 62.96999 37.771273) (width 2) (layer F.Cu) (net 33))
 (segment (start 66.07 39.4) (end 64.598717 39.4) (width 2) (layer F.Cu) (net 33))
 (segment (start 55.19999 47.49999) (end 65.15 57.45) (width 0.25) (layer B.Cu) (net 7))
 (segment (start 57.25 36.63) (end 55.19999 38.68001) (width 0.25) (layer B.Cu) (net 7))
 (segment (start 55.19999 38.68001) (end 55.19999 47.49999) (width 0.25) (layer B.Cu) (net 7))
 (segment (start 57.25 34.09) (end 54.74998 36.59002) (width 0.25) (layer B.Cu) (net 6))
 (segment (start 54.74998 52.19998) (end 60.7 58.15) (width 0.25) (layer B.Cu) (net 6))
 (segment (start 54.74998 36.59002) (end 54.74998 52.19998) (width 0.25) (layer B.Cu) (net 6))
 (segment (start 49.93 36.86) (end 50.83 36.86) (width 0.25) (layer F.Cu) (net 21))
 (segment (start 50.83 26.7) (end 49.93 26.7) (width 0.25) (layer F.Cu) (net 21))
 (segment (start 51.73 36.86) (end 50.83 36.86) (width 0.25) (layer F.Cu) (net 21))
 (segment (start 59.79 31.55) (end 57.69 29.45) (width 0.25) (layer F.Cu) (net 21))
 (segment (start 57.69 29.45) (end 57.69 29.45) (width 0.25) (layer F.Cu) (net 21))
 (via (at 57.69 29.45) (size 0.8) (drill 0.4) (layers F.Cu B.Cu) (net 21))
 (segment (start 51.73 26.7) (end 50.83 26.7) (width 0.25) (layer B.Cu) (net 21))
 (segment (start 54.48 29.45) (end 54.48 29.45) (width 0.25) (layer B.Cu) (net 21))
 (segment (start 57.69 29.45) (end 54.48 29.45) (width 0.25) (layer B.Cu) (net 21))
 (segment (start 54.48 29.45) (end 51.73 26.7) (width 0.25) (layer B.Cu) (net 21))
 (via (at 54.48 29.45) (size 0.8) (drill 0.4) (layers F.Cu B.Cu) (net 21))
 (segment (start 53.374999 33.225001) (end 54.48 32.12) (width 0.25) (layer F.Cu) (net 21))
 (segment (start 53.374999 36.465001) (end 53.374999 33.225001) (width 0.25) (layer F.Cu) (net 21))
 (segment (start 50.83 36.86) (end 52.98 36.86) (width 0.25) (layer F.Cu) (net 21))
 (segment (start 54.48 32.12) (end 54.48 29.45) (width 0.25) (layer F.Cu) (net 21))
 (segment (start 52.98 36.86) (end 53.374999 36.465001) (width 0.25) (layer F.Cu) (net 21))
 (segment (start 52.98 29.24) (end 53.89 30.15) (width 0.25) (layer B.Cu) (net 16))
 (segment (start 50.83 29.24) (end 52.98 29.24) (width 0.25) (layer B.Cu) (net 16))
 (segment (start 53.89 30.15) (end 59.55 30.15) (width 0.25) (layer B.Cu) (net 16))
 (segment (start 59.55 30.15) (end 59.55 30.15) (width 0.25) (layer B.Cu) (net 16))
 (via (at 59.55 30.15) (size 0.8) (drill 0.4) (layers F.Cu B.Cu) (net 16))
 (segment (start 57.25 27.85) (end 57.25 27.49) (width 0.25) (layer F.Cu) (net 16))
 (segment (start 59.55 30.15) (end 57.25 27.85) (width 0.25) (layer F.Cu) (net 16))
 (segment (start 53.05501 30.56501) (end 51.73 29.24) (width 0.25) (layer B.Cu) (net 16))
 (segment (start 53.05501 32.99499) (end 53.05501 30.56501) (width 0.25) (layer B.Cu) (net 16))
 (segment (start 51.73 34.32) (end 53.05501 32.99499) (width 0.25) (layer B.Cu) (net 16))
 (segment (start 51.73 29.24) (end 50.83 29.24) (width 0.25) (layer B.Cu) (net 16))
 (segment (start 50.83 34.32) (end 51.73 34.32) (width 0.25) (layer B.Cu) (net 16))
 (segment (start 26.779999 54.020001) (end 25.78 55.02) (width 0.25) (layer F.Cu) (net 23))
 (segment (start 31.074999 49.725001) (end 26.779999 54.020001) (width 0.25) (layer F.Cu) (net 23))
 (segment (start 31.074999 40.345001) (end 31.074999 49.725001) (width 0.25) (layer F.Cu) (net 23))
 (segment (start 32.25 39.17) (end 31.074999 40.345001) (width 0.25) (layer F.Cu) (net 23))
 (segment (start 40.020001 56.560001) (end 41.02 57.56) (width 0.25) (layer F.Cu) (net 24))
 (segment (start 37.95 54.49) (end 40.020001 56.560001) (width 0.25) (layer F.Cu) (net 24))
 (segment (start 37.95 39.79) (end 37.95 54.49) (width 0.25) (layer F.Cu) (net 24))
 (segment (start 34.79 36.63) (end 37.95 39.79) (width 0.25) (layer F.Cu) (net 24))
 (segment (start 57.25 42.51) (end 57.25 41.71) (width 0.25) (layer F.Cu) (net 13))
 (segment (start 49.9 49.86) (end 57.25 42.51) (width 0.25) (layer F.Cu) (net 13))
 (segment (start 57.25 39.17) (end 55.65 40.77) (width 0.25) (layer B.Cu) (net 8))
 (segment (start 59.63934 46.7) (end 60.7 46.7) (width 0.25) (layer B.Cu) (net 8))
 (segment (start 55.65 42.71066) (end 59.63934 46.7) (width 0.25) (layer B.Cu) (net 8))
 (segment (start 55.65 40.77) (end 55.65 42.71066) (width 0.25) (layer B.Cu) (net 8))
 (segment (start 31.97499 24.67499) (end 32.25 24.95) (width 0.25) (layer B.Cu) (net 4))
 (segment (start 27.873956 24.67499) (end 31.97499 24.67499) (width 0.25) (layer B.Cu) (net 4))
 (segment (start 26.779999 25.768947) (end 27.873956 24.67499) (width 0.25) (layer B.Cu) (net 4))
 (segment (start 26.779999 26.080001) (end 26.779999 25.768947) (width 0.25) (layer B.Cu) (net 4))
 (segment (start 25.78 27.08) (end 26.779999 26.080001) (width 0.25) (layer B.Cu) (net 4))
 (segment (start 27.62499 28.92499) (end 27.62499 36.37499) (width 0.25) (layer B.Cu) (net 4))
 (segment (start 25.78 27.08) (end 27.62499 28.92499) (width 0.25) (layer B.Cu) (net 4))
 (segment (start 29.055001 37.805001) (end 27.62499 36.37499) (width 0.25) (layer B.Cu) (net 4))
 (segment (start 33.425001 37.805001) (end 29.055001 37.805001) (width 0.25) (layer B.Cu) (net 4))
 (segment (start 34.79 39.17) (end 33.425001 37.805001) (width 0.25) (layer B.Cu) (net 4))
 (segment (start 51.73 31.78) (end 50.83 31.78) (width 0.25) (layer F.Cu) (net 18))
 (segment (start 53.05501 30.45499) (end 51.73 31.78) (width 0.25) (layer F.Cu) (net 18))
 (segment (start 51.063847 24.16) (end 53.05501 26.151163) (width 0.25) (layer F.Cu) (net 18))
 (segment (start 53.05501 26.151163) (end 53.05501 30.45499) (width 0.25) (layer F.Cu) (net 18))
 (segment (start 50.83 24.16) (end 51.063847 24.16) (width 0.25) (layer F.Cu) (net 18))
 (segment (start 55.624989 25.475011) (end 56.15 24.95) (width 0.25) (layer F.Cu) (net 18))
 (segment (start 51.224989 39.4) (end 55.624989 35) (width 0.25) (layer F.Cu) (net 18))
 (segment (start 56.15 24.95) (end 57.25 24.95) (width 0.25) (layer F.Cu) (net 18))
 (segment (start 55.624989 35) (end 55.624989 25.475011) (width 0.25) (layer F.Cu) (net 18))
 (segment (start 50.83 39.4) (end 51.224989 39.4) (width 0.25) (layer F.Cu) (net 18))
 (segment (start 60.44 21.94987) (end 60.44 20.65) (width 2) (layer F.Cu) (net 15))
 (segment (start 61.840001 23.349871) (end 60.44 21.94987) (width 2) (layer F.Cu) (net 15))
 (segment (start 61.840001 26.481284) (end 61.840001 23.349871) (width 2) (layer F.Cu) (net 15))
 (segment (start 64.598717 29.24) (end 61.840001 26.481284) (width 2) (layer F.Cu) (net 15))
 (segment (start 66.07 29.24) (end 64.598717 29.24) (width 2) (layer F.Cu) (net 15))
 (segment (start 61.840001 26.64208) (end 61.840001 26.481284) (width 2) (layer F.Cu) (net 15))
 (segment (start 60.992081 27.49) (end 61.840001 26.64208) (width 2) (layer F.Cu) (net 15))
 (segment (start 59.79 27.49) (end 60.992081 27.49) (width 2) (layer F.Cu) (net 15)))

